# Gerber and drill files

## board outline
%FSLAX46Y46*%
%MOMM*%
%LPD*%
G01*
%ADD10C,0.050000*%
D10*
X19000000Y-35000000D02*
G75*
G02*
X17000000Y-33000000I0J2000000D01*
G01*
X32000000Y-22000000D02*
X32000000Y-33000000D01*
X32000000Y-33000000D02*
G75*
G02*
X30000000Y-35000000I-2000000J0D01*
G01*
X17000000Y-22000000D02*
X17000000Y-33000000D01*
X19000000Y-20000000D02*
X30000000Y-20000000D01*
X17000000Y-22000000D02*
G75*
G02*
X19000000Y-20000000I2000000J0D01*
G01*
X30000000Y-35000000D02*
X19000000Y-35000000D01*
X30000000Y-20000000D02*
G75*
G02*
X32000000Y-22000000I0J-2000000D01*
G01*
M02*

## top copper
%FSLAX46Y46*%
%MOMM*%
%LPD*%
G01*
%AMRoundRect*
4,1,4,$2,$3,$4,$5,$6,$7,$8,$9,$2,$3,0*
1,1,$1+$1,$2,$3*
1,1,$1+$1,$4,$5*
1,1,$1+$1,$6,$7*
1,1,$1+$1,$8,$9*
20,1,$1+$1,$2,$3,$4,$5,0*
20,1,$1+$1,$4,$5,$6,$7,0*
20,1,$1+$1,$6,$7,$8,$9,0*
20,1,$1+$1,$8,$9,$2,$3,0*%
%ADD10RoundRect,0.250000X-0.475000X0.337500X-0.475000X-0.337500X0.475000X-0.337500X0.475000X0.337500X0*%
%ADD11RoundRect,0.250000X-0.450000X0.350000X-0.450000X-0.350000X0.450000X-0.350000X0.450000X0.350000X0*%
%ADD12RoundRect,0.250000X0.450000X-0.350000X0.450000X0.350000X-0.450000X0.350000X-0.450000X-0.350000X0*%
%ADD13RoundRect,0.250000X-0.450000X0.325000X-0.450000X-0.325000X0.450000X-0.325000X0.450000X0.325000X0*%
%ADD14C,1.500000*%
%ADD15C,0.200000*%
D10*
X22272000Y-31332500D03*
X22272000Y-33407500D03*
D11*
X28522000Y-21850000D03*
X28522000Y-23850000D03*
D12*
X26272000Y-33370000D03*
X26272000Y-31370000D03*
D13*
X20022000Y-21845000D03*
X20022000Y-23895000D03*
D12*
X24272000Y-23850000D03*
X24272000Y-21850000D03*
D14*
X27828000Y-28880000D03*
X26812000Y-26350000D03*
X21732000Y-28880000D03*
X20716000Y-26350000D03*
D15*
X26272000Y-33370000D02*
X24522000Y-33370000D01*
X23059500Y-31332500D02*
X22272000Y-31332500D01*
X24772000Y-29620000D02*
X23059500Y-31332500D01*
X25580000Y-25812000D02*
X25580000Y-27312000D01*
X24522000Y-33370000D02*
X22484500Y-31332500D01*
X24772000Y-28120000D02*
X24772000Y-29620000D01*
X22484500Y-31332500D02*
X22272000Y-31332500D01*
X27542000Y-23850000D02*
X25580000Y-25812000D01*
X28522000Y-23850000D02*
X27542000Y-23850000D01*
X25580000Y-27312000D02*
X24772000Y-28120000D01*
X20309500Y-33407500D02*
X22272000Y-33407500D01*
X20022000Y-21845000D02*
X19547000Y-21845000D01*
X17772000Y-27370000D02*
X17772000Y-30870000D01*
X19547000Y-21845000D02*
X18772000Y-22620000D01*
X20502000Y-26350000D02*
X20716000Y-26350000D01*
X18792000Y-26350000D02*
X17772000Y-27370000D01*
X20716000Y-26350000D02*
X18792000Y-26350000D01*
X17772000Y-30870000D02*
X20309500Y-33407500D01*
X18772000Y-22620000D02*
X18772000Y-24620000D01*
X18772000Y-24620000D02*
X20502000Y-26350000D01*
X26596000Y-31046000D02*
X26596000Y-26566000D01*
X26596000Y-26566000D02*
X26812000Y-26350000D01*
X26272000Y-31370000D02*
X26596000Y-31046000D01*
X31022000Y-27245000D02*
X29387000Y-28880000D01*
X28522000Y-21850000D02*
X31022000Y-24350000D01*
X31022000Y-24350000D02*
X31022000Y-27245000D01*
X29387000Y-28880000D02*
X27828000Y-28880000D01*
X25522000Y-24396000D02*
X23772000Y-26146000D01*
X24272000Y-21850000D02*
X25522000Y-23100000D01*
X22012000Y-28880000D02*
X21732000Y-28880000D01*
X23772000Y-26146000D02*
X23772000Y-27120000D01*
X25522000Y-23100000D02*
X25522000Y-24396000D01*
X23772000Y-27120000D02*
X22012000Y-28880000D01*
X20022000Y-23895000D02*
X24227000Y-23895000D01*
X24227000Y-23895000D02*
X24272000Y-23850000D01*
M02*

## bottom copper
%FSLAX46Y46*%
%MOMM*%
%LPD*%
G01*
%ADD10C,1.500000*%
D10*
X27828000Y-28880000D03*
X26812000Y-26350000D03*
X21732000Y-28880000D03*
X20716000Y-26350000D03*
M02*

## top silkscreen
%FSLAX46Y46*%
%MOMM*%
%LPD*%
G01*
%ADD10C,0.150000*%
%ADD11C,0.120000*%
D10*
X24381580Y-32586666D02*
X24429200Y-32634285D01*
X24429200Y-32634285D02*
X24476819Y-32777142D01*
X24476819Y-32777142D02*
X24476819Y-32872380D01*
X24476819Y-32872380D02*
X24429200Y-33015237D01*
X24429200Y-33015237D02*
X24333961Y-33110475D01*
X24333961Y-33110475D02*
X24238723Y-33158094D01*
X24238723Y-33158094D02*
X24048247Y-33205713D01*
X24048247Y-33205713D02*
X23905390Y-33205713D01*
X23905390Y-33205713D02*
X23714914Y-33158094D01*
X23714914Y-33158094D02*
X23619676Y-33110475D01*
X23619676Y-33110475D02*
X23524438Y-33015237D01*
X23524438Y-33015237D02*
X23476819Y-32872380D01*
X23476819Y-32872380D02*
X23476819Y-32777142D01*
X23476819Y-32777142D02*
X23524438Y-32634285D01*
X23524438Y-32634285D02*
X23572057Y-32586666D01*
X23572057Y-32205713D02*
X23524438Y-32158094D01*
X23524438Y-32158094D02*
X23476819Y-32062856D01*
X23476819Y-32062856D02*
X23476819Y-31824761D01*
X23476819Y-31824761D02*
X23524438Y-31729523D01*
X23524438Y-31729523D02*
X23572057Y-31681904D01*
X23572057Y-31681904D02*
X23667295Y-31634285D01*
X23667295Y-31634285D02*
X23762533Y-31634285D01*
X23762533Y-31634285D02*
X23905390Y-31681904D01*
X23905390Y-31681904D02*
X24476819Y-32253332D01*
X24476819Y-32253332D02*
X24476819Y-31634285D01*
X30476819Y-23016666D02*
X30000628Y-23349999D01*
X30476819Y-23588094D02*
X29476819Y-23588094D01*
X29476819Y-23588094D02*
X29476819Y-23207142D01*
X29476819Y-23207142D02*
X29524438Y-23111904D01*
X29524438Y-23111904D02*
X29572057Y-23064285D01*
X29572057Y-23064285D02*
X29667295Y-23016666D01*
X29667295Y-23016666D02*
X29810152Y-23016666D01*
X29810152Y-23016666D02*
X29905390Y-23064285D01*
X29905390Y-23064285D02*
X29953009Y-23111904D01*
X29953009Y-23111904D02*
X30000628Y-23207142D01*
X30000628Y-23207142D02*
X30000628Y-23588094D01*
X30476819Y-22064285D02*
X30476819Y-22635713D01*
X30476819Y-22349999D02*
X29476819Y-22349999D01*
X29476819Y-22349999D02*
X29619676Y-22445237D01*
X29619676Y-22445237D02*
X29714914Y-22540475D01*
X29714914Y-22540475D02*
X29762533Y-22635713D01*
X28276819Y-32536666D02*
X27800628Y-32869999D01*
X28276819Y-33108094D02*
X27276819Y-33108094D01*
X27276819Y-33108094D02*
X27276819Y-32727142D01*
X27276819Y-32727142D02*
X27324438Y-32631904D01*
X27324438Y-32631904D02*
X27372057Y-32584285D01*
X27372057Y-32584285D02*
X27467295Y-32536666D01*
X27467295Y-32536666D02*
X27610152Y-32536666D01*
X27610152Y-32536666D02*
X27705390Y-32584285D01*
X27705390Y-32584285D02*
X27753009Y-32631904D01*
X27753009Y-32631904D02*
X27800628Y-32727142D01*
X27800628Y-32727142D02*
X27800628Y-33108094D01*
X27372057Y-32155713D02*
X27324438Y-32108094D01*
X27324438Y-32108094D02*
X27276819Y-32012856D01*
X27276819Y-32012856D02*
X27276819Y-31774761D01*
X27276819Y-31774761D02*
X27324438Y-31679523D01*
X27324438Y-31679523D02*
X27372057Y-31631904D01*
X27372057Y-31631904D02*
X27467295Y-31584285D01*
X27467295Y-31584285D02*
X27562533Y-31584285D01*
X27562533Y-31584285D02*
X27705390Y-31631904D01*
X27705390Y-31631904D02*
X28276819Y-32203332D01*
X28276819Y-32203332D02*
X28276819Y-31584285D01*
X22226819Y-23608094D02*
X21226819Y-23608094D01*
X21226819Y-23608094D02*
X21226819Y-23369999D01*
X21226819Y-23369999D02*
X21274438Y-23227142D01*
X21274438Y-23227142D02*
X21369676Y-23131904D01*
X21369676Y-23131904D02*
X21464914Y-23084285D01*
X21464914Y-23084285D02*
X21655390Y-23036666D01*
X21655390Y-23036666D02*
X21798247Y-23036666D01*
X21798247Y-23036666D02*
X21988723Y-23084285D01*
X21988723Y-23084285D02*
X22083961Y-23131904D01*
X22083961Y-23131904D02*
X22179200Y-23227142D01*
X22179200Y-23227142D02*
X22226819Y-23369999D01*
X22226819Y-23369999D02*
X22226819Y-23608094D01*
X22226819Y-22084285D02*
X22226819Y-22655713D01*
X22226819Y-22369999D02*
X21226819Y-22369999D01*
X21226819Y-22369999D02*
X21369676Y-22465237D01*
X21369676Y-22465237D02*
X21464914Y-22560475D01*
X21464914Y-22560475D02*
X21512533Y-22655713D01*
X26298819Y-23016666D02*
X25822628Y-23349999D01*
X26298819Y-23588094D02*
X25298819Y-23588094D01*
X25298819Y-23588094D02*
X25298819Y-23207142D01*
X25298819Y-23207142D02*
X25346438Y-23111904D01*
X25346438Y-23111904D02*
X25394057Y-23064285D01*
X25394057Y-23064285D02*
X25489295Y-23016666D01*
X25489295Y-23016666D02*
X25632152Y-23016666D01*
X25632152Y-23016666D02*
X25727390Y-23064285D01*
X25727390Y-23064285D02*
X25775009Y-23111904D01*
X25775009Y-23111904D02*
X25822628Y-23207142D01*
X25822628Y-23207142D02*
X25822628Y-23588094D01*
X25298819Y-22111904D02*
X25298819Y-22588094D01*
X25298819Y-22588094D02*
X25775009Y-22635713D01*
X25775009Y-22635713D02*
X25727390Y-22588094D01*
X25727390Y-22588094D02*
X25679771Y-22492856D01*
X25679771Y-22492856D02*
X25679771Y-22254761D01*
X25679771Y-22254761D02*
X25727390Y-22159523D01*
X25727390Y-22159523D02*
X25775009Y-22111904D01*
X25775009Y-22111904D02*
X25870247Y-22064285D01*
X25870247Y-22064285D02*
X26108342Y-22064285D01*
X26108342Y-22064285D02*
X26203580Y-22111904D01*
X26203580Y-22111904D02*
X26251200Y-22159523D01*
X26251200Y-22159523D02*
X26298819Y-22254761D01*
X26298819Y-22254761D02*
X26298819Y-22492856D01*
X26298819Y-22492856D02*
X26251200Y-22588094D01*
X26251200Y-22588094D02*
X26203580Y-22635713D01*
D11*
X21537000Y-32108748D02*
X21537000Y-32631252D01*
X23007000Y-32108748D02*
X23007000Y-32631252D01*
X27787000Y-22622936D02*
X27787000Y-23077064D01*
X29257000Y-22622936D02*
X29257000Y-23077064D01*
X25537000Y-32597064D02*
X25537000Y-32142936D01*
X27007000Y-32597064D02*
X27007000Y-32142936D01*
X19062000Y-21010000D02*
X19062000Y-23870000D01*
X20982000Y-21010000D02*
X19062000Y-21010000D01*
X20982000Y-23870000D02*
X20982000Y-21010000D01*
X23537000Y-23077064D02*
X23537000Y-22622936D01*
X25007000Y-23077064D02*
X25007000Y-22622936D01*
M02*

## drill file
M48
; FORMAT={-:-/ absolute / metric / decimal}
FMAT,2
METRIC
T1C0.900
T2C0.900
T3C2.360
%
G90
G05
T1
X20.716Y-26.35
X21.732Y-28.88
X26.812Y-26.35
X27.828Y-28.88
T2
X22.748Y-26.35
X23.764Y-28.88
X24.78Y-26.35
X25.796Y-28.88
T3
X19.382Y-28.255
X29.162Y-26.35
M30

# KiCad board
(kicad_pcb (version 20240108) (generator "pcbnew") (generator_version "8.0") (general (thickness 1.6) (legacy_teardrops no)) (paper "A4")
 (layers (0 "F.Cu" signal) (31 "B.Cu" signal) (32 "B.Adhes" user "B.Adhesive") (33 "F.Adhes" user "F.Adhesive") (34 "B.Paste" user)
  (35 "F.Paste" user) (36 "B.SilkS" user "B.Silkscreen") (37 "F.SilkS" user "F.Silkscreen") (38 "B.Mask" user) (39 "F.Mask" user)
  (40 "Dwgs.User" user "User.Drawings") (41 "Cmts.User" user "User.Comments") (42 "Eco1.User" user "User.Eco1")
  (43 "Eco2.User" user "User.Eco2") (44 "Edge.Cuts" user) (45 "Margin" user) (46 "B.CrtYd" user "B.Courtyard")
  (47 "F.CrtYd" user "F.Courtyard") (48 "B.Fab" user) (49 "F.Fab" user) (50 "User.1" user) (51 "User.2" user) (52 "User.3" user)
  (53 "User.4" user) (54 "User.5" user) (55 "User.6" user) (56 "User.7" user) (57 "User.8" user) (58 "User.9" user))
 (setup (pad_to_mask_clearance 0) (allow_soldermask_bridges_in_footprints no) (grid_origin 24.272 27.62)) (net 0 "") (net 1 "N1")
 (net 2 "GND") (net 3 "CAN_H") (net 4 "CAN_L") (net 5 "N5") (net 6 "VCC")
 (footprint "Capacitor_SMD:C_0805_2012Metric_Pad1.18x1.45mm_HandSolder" (layer "F.Cu") (at 22.272 32.37 -90)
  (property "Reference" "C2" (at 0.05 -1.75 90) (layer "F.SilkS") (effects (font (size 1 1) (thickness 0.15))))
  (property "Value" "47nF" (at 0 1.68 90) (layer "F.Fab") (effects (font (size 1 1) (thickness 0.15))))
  (fp_line (start -0.261252 0.735) (end 0.261252 0.735) (stroke (width 0.12) (type solid)) (layer "F.SilkS"))
  (fp_line (start -0.261252 -0.735) (end 0.261252 -0.735) (stroke (width 0.12) (type solid)) (layer "F.SilkS"))
  (pad "1" smd roundrect (at -1.0375 0 270) (size 1.175 1.45) (layers "F.Cu" "F.Paste" "F.Mask") (roundrect_rratio 0.212766) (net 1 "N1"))
  (pad "2" smd roundrect (at 1.0375 0 270) (size 1.175 1.45) (layers "F.Cu" "F.Paste" "F.Mask") (roundrect_rratio 0.212766) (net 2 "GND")))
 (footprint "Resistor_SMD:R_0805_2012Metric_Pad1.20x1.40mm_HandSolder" (layer "F.Cu") (at 28.522 22.85 -90)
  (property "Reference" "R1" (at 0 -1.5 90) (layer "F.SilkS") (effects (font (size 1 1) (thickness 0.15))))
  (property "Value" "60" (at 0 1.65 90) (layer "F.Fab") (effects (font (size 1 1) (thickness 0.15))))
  (fp_line (start -0.227064 0.735) (end 0.227064 0.735) (stroke (width 0.12) (type solid)) (layer "F.SilkS"))
  (fp_line (start -0.227064 -0.735) (end 0.227064 -0.735) (stroke (width 0.12) (type solid)) (layer "F.SilkS"))
  (pad "1" smd roundrect (at -1 0 270) (size 1.2 1.4) (layers "F.Cu" "F.Paste" "F.Mask") (roundrect_rratio 0.208333) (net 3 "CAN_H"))
  (pad "2" smd roundrect (at 1 0 270) (size 1.2 1.4) (layers "F.Cu" "F.Paste" "F.Mask") (roundrect_rratio 0.208333) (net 1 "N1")))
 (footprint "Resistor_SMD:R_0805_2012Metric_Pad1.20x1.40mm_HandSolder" (layer "F.Cu") (at 26.272 32.37 90)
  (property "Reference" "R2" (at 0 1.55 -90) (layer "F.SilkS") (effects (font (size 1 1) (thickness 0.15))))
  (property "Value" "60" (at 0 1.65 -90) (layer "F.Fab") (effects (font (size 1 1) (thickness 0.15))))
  (fp_line (start -0.227064 -0.735) (end 0.227064 -0.735) (stroke (width 0.12) (type solid)) (layer "F.SilkS"))
  (fp_line (start -0.227064 0.735) (end 0.227064 0.735) (stroke (width 0.12) (type solid)) (layer "F.SilkS"))
  (pad "1" smd roundrect (at -1 0 90) (size 1.2 1.4) (layers "F.Cu" "F.Paste" "F.Mask") (roundrect_rratio 0.208333) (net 1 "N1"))
  (pad "2" smd roundrect (at 1 0 90) (size 1.2 1.4) (layers "F.Cu" "F.Paste" "F.Mask") (roundrect_rratio 0.208333) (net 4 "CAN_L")))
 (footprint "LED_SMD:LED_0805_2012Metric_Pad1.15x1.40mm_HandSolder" (layer "F.Cu") (at 20.022 22.87 -90)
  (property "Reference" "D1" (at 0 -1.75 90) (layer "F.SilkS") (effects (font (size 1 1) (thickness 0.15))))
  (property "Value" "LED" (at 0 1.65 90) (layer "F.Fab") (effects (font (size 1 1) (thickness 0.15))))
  (fp_line (start -1.86 0.96) (end 1 0.96) (stroke (width 0.12) (type solid)) (layer "F.SilkS"))
  (fp_line (start -1.86 -0.96) (end -1.86 0.96) (stroke (width 0.12) (type solid)) (layer "F.SilkS"))
  (fp_line (start 1 -0.96) (end -1.86 -0.96) (stroke (width 0.12) (type solid)) (layer "F.SilkS"))
  (pad "1" smd roundrect (at -1.025 0 270) (size 1.15 1.4) (layers "F.Cu" "F.Paste" "F.Mask") (roundrect_rratio 0.217391) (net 2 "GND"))
  (pad "2" smd roundrect (at 1.025 0 270) (size 1.15 1.4) (layers "F.Cu" "F.Paste" "F.Mask") (roundrect_rratio 0.217391) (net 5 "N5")))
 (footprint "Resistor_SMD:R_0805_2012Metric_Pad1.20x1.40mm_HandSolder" (layer "F.Cu") (at 24.272 22.85 90)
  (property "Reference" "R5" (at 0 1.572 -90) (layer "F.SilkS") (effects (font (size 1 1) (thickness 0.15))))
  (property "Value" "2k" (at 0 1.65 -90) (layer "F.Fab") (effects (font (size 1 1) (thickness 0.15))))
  (fp_line (start -0.227064 -0.735) (end 0.227064 -0.735) (stroke (width 0.12) (type solid)) (layer "F.SilkS"))
  (fp_line (start -0.227064 0.735) (end 0.227064 0.735) (stroke (width 0.12) (type solid)) (layer "F.SilkS"))
  (pad "1" smd roundrect (at -1 0 90) (size 1.2 1.4) (layers "F.Cu" "F.Paste" "F.Mask") (roundrect_rratio 0.208333) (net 5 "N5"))
  (pad "2" smd roundrect (at 1 0 90) (size 1.2 1.4) (layers "F.Cu" "F.Paste" "F.Mask") (roundrect_rratio 0.208333) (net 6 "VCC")))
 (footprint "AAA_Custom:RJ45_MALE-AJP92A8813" (layer "B.Cu") (at 24.272 27.62 180)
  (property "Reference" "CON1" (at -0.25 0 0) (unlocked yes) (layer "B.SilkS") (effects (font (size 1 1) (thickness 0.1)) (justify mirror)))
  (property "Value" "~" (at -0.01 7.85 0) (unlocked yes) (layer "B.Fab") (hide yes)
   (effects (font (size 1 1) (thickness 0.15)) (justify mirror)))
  (pad "" np_thru_hole circle (at -4.89 1.27 180) (size 2.3 2.3) (drill 2.36) (layers "F&B.Cu" "*.Mask"))
  (pad "" np_thru_hole circle (at -1.524 -1.26 180) (size 0.2 0.2) (drill 0.9) (layers "F&B.Cu" "*.Mask"))
  (pad "" np_thru_hole circle (at -0.508 1.27 180) (size 0.2 0.2) (drill 0.9) (layers "F&B.Cu" "*.Mask"))
  (pad "" np_thru_hole circle (at 0.508 -1.26 180) (size 0.2 0.2) (drill 0.9) (layers "F&B.Cu" "*.Mask"))
  (pad "" np_thru_hole circle (at 1.524 1.27 180) (size 0.2 0.2) (drill 0.9) (layers "F&B.Cu" "*.Mask"))
  (pad "" np_thru_hole circle (at 4.89 -0.635 180) (size 2.3 2.3) (drill 2.36) (layers "F&B.Cu" "*.Mask"))
  (pad "1" thru_hole circle (at -3.556 -1.26 180) (size 1.5 1.5) (drill 0.9) (layers "*.Cu" "*.Mask") (remove_unused_layers no)
   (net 3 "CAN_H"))
  (pad "2" thru_hole circle (at -2.54 1.27 180) (size 1.5 1.5) (drill 0.9) (layers "*.Cu" "*.Mask") (remove_unused_layers no)
   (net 4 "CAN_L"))
  (pad "7" thru_hole circle (at 2.54 -1.26 180) (size 1.5 1.5) (drill 0.9) (layers "*.Cu" "*.Mask") (remove_unused_layers no) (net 6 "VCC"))
  (pad "8" thru_hole circle (at 3.556 1.27 180) (size 1.5 1.5) (drill 0.9) (layers "*.Cu" "*.Mask") (remove_unused_layers no) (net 2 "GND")))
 (gr_arc (start 19 35) (mid 17.585786 34.414214) (end 17 33) (stroke (width 0.05) (type default)) (layer "Edge.Cuts"))
 (gr_line (start 32 22) (end 32 33) (stroke (width 0.05) (type default)) (layer "Edge.Cuts"))
 (gr_arc (start 32 33) (mid 31.414214 34.414214) (end 30 35) (stroke (width 0.05) (type default)) (layer "Edge.Cuts"))
 (gr_line (start 17 22) (end 17 33) (stroke (width 0.05) (type default)) (layer "Edge.Cuts"))
 (gr_line (start 19 20) (end 30 20) (stroke (width 0.05) (type default)) (layer "Edge.Cuts"))
 (gr_arc (start 17 22) (mid 17.585786 20.585786) (end 19 20) (stroke (width 0.05) (type default)) (layer "Edge.Cuts"))
 (gr_line (start 30 35) (end 19 35) (stroke (width 0.05) (type default)) (layer "Edge.Cuts"))
 (gr_arc (start 30 20) (mid 31.414214 20.585786) (end 32 22) (stroke (width 0.05) (type default)) (layer "Edge.Cuts"))
 (segment (start 26.272 33.37) (end 24.522 33.37) (width 0.2) (layer "F.Cu") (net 1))
 (segment (start 23.0595 31.3325) (end 22.272 31.3325) (width 0.2) (layer "F.Cu") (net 1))
 (segment (start 24.772 29.62) (end 23.0595 31.3325) (width 0.2) (layer "F.Cu") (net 1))
 (segment (start 25.58 25.812) (end 25.58 27.312) (width 0.2) (layer "F.Cu") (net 1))
 (segment (start 24.522 33.37) (end 22.4845 31.3325) (width 0.2) (layer "F.Cu") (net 1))
 (segment (start 24.772 28.12) (end 24.772 29.62) (width 0.2) (layer "F.Cu") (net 1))
 (segment (start 22.4845 31.3325) (end 22.272 31.3325) (width 0.2) (layer "F.Cu") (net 1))
 (segment (start 27.542 23.85) (end 25.58 25.812) (width 0.2) (layer "F.Cu") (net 1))
 (segment (start 28.522 23.85) (end 27.542 23.85) (width 0.2) (layer "F.Cu") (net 1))
 (segment (start 25.58 27.312) (end 24.772 28.12) (width 0.2) (layer "F.Cu") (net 1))
 (segment (start 20.3095 33.4075) (end 22.272 33.4075) (width 0.2) (layer "F.Cu") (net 2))
 (segment (start 20.022 21.845) (end 19.547 21.845) (width 0.2) (layer "F.Cu") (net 2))
 (segment (start 17.772 27.37) (end 17.772 30.87) (width 0.2) (layer "F.Cu") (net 2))
 (segment (start 19.547 21.845) (end 18.772 22.62) (width 0.2) (layer "F.Cu") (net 2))
 (segment (start 20.502 26.35) (end 20.716 26.35) (width 0.2) (layer "F.Cu") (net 2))
 (segment (start 18.792 26.35) (end 17.772 27.37) (width 0.2) (layer "F.Cu") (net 2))
 (segment (start 20.716 26.35) (end 18.792 26.35) (width 0.2) (layer "F.Cu") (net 2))
 (segment (start 17.772 30.87) (end 20.3095 33.4075) (width 0.2) (layer "F.Cu") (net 2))
 (segment (start 18.772 22.62) (end 18.772 24.62) (width 0.2) (layer "F.Cu") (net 2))
 (segment (start 18.772 24.62) (end 20.502 26.35) (width 0.2) (layer "F.Cu") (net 2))
 (segment (start 26.596 31.046) (end 26.596 26.566) (width 0.2) (layer "F.Cu") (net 4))
 (segment (start 26.596 26.566) (end 26.812 26.35) (width 0.2) (layer "F.Cu") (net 4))
 (segment (start 26.272 31.37) (end 26.596 31.046) (width 0.2) (layer "F.Cu") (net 4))
 (segment (start 31.022 27.245) (end 29.387 28.88) (width 0.2) (layer "F.Cu") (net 3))
 (segment (start 28.522 21.85) (end 31.022 24.35) (width 0.2) (layer "F.Cu") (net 3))
 (segment (start 31.022 24.35) (end 31.022 27.245) (width 0.2) (layer "F.Cu") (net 3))
 (segment (start 29.387 28.88) (end 27.828 28.88) (width 0.2) (layer "F.Cu") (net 3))
 (segment (start 25.522 24.396) (end 23.772 26.146) (width 0.2) (layer "F.Cu") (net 6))
 (segment (start 24.272 21.85) (end 25.522 23.1) (width 0.2) (layer "F.Cu") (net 6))
 (segment (start 22.012 28.88) (end 21.732 28.88) (width 0.2) (layer "F.Cu") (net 6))
 (segment (start 23.772 26.146) (end 23.772 27.12) (width 0.2) (layer "F.Cu") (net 6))
 (segment (start 25.522 23.1) (end 25.522 24.396) (width 0.2) (layer "F.Cu") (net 6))
 (segment (start 23.772 27.12) (end 22.012 28.88) (width 0.2) (layer "F.Cu") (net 6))
 (segment (start 20.022 23.895) (end 24.227 23.895) (width 0.2) (layer "F.Cu") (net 5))
 (segment (start 24.227 23.895) (end 24.272 23.85) (width 0.2) (layer "F.Cu") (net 5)))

